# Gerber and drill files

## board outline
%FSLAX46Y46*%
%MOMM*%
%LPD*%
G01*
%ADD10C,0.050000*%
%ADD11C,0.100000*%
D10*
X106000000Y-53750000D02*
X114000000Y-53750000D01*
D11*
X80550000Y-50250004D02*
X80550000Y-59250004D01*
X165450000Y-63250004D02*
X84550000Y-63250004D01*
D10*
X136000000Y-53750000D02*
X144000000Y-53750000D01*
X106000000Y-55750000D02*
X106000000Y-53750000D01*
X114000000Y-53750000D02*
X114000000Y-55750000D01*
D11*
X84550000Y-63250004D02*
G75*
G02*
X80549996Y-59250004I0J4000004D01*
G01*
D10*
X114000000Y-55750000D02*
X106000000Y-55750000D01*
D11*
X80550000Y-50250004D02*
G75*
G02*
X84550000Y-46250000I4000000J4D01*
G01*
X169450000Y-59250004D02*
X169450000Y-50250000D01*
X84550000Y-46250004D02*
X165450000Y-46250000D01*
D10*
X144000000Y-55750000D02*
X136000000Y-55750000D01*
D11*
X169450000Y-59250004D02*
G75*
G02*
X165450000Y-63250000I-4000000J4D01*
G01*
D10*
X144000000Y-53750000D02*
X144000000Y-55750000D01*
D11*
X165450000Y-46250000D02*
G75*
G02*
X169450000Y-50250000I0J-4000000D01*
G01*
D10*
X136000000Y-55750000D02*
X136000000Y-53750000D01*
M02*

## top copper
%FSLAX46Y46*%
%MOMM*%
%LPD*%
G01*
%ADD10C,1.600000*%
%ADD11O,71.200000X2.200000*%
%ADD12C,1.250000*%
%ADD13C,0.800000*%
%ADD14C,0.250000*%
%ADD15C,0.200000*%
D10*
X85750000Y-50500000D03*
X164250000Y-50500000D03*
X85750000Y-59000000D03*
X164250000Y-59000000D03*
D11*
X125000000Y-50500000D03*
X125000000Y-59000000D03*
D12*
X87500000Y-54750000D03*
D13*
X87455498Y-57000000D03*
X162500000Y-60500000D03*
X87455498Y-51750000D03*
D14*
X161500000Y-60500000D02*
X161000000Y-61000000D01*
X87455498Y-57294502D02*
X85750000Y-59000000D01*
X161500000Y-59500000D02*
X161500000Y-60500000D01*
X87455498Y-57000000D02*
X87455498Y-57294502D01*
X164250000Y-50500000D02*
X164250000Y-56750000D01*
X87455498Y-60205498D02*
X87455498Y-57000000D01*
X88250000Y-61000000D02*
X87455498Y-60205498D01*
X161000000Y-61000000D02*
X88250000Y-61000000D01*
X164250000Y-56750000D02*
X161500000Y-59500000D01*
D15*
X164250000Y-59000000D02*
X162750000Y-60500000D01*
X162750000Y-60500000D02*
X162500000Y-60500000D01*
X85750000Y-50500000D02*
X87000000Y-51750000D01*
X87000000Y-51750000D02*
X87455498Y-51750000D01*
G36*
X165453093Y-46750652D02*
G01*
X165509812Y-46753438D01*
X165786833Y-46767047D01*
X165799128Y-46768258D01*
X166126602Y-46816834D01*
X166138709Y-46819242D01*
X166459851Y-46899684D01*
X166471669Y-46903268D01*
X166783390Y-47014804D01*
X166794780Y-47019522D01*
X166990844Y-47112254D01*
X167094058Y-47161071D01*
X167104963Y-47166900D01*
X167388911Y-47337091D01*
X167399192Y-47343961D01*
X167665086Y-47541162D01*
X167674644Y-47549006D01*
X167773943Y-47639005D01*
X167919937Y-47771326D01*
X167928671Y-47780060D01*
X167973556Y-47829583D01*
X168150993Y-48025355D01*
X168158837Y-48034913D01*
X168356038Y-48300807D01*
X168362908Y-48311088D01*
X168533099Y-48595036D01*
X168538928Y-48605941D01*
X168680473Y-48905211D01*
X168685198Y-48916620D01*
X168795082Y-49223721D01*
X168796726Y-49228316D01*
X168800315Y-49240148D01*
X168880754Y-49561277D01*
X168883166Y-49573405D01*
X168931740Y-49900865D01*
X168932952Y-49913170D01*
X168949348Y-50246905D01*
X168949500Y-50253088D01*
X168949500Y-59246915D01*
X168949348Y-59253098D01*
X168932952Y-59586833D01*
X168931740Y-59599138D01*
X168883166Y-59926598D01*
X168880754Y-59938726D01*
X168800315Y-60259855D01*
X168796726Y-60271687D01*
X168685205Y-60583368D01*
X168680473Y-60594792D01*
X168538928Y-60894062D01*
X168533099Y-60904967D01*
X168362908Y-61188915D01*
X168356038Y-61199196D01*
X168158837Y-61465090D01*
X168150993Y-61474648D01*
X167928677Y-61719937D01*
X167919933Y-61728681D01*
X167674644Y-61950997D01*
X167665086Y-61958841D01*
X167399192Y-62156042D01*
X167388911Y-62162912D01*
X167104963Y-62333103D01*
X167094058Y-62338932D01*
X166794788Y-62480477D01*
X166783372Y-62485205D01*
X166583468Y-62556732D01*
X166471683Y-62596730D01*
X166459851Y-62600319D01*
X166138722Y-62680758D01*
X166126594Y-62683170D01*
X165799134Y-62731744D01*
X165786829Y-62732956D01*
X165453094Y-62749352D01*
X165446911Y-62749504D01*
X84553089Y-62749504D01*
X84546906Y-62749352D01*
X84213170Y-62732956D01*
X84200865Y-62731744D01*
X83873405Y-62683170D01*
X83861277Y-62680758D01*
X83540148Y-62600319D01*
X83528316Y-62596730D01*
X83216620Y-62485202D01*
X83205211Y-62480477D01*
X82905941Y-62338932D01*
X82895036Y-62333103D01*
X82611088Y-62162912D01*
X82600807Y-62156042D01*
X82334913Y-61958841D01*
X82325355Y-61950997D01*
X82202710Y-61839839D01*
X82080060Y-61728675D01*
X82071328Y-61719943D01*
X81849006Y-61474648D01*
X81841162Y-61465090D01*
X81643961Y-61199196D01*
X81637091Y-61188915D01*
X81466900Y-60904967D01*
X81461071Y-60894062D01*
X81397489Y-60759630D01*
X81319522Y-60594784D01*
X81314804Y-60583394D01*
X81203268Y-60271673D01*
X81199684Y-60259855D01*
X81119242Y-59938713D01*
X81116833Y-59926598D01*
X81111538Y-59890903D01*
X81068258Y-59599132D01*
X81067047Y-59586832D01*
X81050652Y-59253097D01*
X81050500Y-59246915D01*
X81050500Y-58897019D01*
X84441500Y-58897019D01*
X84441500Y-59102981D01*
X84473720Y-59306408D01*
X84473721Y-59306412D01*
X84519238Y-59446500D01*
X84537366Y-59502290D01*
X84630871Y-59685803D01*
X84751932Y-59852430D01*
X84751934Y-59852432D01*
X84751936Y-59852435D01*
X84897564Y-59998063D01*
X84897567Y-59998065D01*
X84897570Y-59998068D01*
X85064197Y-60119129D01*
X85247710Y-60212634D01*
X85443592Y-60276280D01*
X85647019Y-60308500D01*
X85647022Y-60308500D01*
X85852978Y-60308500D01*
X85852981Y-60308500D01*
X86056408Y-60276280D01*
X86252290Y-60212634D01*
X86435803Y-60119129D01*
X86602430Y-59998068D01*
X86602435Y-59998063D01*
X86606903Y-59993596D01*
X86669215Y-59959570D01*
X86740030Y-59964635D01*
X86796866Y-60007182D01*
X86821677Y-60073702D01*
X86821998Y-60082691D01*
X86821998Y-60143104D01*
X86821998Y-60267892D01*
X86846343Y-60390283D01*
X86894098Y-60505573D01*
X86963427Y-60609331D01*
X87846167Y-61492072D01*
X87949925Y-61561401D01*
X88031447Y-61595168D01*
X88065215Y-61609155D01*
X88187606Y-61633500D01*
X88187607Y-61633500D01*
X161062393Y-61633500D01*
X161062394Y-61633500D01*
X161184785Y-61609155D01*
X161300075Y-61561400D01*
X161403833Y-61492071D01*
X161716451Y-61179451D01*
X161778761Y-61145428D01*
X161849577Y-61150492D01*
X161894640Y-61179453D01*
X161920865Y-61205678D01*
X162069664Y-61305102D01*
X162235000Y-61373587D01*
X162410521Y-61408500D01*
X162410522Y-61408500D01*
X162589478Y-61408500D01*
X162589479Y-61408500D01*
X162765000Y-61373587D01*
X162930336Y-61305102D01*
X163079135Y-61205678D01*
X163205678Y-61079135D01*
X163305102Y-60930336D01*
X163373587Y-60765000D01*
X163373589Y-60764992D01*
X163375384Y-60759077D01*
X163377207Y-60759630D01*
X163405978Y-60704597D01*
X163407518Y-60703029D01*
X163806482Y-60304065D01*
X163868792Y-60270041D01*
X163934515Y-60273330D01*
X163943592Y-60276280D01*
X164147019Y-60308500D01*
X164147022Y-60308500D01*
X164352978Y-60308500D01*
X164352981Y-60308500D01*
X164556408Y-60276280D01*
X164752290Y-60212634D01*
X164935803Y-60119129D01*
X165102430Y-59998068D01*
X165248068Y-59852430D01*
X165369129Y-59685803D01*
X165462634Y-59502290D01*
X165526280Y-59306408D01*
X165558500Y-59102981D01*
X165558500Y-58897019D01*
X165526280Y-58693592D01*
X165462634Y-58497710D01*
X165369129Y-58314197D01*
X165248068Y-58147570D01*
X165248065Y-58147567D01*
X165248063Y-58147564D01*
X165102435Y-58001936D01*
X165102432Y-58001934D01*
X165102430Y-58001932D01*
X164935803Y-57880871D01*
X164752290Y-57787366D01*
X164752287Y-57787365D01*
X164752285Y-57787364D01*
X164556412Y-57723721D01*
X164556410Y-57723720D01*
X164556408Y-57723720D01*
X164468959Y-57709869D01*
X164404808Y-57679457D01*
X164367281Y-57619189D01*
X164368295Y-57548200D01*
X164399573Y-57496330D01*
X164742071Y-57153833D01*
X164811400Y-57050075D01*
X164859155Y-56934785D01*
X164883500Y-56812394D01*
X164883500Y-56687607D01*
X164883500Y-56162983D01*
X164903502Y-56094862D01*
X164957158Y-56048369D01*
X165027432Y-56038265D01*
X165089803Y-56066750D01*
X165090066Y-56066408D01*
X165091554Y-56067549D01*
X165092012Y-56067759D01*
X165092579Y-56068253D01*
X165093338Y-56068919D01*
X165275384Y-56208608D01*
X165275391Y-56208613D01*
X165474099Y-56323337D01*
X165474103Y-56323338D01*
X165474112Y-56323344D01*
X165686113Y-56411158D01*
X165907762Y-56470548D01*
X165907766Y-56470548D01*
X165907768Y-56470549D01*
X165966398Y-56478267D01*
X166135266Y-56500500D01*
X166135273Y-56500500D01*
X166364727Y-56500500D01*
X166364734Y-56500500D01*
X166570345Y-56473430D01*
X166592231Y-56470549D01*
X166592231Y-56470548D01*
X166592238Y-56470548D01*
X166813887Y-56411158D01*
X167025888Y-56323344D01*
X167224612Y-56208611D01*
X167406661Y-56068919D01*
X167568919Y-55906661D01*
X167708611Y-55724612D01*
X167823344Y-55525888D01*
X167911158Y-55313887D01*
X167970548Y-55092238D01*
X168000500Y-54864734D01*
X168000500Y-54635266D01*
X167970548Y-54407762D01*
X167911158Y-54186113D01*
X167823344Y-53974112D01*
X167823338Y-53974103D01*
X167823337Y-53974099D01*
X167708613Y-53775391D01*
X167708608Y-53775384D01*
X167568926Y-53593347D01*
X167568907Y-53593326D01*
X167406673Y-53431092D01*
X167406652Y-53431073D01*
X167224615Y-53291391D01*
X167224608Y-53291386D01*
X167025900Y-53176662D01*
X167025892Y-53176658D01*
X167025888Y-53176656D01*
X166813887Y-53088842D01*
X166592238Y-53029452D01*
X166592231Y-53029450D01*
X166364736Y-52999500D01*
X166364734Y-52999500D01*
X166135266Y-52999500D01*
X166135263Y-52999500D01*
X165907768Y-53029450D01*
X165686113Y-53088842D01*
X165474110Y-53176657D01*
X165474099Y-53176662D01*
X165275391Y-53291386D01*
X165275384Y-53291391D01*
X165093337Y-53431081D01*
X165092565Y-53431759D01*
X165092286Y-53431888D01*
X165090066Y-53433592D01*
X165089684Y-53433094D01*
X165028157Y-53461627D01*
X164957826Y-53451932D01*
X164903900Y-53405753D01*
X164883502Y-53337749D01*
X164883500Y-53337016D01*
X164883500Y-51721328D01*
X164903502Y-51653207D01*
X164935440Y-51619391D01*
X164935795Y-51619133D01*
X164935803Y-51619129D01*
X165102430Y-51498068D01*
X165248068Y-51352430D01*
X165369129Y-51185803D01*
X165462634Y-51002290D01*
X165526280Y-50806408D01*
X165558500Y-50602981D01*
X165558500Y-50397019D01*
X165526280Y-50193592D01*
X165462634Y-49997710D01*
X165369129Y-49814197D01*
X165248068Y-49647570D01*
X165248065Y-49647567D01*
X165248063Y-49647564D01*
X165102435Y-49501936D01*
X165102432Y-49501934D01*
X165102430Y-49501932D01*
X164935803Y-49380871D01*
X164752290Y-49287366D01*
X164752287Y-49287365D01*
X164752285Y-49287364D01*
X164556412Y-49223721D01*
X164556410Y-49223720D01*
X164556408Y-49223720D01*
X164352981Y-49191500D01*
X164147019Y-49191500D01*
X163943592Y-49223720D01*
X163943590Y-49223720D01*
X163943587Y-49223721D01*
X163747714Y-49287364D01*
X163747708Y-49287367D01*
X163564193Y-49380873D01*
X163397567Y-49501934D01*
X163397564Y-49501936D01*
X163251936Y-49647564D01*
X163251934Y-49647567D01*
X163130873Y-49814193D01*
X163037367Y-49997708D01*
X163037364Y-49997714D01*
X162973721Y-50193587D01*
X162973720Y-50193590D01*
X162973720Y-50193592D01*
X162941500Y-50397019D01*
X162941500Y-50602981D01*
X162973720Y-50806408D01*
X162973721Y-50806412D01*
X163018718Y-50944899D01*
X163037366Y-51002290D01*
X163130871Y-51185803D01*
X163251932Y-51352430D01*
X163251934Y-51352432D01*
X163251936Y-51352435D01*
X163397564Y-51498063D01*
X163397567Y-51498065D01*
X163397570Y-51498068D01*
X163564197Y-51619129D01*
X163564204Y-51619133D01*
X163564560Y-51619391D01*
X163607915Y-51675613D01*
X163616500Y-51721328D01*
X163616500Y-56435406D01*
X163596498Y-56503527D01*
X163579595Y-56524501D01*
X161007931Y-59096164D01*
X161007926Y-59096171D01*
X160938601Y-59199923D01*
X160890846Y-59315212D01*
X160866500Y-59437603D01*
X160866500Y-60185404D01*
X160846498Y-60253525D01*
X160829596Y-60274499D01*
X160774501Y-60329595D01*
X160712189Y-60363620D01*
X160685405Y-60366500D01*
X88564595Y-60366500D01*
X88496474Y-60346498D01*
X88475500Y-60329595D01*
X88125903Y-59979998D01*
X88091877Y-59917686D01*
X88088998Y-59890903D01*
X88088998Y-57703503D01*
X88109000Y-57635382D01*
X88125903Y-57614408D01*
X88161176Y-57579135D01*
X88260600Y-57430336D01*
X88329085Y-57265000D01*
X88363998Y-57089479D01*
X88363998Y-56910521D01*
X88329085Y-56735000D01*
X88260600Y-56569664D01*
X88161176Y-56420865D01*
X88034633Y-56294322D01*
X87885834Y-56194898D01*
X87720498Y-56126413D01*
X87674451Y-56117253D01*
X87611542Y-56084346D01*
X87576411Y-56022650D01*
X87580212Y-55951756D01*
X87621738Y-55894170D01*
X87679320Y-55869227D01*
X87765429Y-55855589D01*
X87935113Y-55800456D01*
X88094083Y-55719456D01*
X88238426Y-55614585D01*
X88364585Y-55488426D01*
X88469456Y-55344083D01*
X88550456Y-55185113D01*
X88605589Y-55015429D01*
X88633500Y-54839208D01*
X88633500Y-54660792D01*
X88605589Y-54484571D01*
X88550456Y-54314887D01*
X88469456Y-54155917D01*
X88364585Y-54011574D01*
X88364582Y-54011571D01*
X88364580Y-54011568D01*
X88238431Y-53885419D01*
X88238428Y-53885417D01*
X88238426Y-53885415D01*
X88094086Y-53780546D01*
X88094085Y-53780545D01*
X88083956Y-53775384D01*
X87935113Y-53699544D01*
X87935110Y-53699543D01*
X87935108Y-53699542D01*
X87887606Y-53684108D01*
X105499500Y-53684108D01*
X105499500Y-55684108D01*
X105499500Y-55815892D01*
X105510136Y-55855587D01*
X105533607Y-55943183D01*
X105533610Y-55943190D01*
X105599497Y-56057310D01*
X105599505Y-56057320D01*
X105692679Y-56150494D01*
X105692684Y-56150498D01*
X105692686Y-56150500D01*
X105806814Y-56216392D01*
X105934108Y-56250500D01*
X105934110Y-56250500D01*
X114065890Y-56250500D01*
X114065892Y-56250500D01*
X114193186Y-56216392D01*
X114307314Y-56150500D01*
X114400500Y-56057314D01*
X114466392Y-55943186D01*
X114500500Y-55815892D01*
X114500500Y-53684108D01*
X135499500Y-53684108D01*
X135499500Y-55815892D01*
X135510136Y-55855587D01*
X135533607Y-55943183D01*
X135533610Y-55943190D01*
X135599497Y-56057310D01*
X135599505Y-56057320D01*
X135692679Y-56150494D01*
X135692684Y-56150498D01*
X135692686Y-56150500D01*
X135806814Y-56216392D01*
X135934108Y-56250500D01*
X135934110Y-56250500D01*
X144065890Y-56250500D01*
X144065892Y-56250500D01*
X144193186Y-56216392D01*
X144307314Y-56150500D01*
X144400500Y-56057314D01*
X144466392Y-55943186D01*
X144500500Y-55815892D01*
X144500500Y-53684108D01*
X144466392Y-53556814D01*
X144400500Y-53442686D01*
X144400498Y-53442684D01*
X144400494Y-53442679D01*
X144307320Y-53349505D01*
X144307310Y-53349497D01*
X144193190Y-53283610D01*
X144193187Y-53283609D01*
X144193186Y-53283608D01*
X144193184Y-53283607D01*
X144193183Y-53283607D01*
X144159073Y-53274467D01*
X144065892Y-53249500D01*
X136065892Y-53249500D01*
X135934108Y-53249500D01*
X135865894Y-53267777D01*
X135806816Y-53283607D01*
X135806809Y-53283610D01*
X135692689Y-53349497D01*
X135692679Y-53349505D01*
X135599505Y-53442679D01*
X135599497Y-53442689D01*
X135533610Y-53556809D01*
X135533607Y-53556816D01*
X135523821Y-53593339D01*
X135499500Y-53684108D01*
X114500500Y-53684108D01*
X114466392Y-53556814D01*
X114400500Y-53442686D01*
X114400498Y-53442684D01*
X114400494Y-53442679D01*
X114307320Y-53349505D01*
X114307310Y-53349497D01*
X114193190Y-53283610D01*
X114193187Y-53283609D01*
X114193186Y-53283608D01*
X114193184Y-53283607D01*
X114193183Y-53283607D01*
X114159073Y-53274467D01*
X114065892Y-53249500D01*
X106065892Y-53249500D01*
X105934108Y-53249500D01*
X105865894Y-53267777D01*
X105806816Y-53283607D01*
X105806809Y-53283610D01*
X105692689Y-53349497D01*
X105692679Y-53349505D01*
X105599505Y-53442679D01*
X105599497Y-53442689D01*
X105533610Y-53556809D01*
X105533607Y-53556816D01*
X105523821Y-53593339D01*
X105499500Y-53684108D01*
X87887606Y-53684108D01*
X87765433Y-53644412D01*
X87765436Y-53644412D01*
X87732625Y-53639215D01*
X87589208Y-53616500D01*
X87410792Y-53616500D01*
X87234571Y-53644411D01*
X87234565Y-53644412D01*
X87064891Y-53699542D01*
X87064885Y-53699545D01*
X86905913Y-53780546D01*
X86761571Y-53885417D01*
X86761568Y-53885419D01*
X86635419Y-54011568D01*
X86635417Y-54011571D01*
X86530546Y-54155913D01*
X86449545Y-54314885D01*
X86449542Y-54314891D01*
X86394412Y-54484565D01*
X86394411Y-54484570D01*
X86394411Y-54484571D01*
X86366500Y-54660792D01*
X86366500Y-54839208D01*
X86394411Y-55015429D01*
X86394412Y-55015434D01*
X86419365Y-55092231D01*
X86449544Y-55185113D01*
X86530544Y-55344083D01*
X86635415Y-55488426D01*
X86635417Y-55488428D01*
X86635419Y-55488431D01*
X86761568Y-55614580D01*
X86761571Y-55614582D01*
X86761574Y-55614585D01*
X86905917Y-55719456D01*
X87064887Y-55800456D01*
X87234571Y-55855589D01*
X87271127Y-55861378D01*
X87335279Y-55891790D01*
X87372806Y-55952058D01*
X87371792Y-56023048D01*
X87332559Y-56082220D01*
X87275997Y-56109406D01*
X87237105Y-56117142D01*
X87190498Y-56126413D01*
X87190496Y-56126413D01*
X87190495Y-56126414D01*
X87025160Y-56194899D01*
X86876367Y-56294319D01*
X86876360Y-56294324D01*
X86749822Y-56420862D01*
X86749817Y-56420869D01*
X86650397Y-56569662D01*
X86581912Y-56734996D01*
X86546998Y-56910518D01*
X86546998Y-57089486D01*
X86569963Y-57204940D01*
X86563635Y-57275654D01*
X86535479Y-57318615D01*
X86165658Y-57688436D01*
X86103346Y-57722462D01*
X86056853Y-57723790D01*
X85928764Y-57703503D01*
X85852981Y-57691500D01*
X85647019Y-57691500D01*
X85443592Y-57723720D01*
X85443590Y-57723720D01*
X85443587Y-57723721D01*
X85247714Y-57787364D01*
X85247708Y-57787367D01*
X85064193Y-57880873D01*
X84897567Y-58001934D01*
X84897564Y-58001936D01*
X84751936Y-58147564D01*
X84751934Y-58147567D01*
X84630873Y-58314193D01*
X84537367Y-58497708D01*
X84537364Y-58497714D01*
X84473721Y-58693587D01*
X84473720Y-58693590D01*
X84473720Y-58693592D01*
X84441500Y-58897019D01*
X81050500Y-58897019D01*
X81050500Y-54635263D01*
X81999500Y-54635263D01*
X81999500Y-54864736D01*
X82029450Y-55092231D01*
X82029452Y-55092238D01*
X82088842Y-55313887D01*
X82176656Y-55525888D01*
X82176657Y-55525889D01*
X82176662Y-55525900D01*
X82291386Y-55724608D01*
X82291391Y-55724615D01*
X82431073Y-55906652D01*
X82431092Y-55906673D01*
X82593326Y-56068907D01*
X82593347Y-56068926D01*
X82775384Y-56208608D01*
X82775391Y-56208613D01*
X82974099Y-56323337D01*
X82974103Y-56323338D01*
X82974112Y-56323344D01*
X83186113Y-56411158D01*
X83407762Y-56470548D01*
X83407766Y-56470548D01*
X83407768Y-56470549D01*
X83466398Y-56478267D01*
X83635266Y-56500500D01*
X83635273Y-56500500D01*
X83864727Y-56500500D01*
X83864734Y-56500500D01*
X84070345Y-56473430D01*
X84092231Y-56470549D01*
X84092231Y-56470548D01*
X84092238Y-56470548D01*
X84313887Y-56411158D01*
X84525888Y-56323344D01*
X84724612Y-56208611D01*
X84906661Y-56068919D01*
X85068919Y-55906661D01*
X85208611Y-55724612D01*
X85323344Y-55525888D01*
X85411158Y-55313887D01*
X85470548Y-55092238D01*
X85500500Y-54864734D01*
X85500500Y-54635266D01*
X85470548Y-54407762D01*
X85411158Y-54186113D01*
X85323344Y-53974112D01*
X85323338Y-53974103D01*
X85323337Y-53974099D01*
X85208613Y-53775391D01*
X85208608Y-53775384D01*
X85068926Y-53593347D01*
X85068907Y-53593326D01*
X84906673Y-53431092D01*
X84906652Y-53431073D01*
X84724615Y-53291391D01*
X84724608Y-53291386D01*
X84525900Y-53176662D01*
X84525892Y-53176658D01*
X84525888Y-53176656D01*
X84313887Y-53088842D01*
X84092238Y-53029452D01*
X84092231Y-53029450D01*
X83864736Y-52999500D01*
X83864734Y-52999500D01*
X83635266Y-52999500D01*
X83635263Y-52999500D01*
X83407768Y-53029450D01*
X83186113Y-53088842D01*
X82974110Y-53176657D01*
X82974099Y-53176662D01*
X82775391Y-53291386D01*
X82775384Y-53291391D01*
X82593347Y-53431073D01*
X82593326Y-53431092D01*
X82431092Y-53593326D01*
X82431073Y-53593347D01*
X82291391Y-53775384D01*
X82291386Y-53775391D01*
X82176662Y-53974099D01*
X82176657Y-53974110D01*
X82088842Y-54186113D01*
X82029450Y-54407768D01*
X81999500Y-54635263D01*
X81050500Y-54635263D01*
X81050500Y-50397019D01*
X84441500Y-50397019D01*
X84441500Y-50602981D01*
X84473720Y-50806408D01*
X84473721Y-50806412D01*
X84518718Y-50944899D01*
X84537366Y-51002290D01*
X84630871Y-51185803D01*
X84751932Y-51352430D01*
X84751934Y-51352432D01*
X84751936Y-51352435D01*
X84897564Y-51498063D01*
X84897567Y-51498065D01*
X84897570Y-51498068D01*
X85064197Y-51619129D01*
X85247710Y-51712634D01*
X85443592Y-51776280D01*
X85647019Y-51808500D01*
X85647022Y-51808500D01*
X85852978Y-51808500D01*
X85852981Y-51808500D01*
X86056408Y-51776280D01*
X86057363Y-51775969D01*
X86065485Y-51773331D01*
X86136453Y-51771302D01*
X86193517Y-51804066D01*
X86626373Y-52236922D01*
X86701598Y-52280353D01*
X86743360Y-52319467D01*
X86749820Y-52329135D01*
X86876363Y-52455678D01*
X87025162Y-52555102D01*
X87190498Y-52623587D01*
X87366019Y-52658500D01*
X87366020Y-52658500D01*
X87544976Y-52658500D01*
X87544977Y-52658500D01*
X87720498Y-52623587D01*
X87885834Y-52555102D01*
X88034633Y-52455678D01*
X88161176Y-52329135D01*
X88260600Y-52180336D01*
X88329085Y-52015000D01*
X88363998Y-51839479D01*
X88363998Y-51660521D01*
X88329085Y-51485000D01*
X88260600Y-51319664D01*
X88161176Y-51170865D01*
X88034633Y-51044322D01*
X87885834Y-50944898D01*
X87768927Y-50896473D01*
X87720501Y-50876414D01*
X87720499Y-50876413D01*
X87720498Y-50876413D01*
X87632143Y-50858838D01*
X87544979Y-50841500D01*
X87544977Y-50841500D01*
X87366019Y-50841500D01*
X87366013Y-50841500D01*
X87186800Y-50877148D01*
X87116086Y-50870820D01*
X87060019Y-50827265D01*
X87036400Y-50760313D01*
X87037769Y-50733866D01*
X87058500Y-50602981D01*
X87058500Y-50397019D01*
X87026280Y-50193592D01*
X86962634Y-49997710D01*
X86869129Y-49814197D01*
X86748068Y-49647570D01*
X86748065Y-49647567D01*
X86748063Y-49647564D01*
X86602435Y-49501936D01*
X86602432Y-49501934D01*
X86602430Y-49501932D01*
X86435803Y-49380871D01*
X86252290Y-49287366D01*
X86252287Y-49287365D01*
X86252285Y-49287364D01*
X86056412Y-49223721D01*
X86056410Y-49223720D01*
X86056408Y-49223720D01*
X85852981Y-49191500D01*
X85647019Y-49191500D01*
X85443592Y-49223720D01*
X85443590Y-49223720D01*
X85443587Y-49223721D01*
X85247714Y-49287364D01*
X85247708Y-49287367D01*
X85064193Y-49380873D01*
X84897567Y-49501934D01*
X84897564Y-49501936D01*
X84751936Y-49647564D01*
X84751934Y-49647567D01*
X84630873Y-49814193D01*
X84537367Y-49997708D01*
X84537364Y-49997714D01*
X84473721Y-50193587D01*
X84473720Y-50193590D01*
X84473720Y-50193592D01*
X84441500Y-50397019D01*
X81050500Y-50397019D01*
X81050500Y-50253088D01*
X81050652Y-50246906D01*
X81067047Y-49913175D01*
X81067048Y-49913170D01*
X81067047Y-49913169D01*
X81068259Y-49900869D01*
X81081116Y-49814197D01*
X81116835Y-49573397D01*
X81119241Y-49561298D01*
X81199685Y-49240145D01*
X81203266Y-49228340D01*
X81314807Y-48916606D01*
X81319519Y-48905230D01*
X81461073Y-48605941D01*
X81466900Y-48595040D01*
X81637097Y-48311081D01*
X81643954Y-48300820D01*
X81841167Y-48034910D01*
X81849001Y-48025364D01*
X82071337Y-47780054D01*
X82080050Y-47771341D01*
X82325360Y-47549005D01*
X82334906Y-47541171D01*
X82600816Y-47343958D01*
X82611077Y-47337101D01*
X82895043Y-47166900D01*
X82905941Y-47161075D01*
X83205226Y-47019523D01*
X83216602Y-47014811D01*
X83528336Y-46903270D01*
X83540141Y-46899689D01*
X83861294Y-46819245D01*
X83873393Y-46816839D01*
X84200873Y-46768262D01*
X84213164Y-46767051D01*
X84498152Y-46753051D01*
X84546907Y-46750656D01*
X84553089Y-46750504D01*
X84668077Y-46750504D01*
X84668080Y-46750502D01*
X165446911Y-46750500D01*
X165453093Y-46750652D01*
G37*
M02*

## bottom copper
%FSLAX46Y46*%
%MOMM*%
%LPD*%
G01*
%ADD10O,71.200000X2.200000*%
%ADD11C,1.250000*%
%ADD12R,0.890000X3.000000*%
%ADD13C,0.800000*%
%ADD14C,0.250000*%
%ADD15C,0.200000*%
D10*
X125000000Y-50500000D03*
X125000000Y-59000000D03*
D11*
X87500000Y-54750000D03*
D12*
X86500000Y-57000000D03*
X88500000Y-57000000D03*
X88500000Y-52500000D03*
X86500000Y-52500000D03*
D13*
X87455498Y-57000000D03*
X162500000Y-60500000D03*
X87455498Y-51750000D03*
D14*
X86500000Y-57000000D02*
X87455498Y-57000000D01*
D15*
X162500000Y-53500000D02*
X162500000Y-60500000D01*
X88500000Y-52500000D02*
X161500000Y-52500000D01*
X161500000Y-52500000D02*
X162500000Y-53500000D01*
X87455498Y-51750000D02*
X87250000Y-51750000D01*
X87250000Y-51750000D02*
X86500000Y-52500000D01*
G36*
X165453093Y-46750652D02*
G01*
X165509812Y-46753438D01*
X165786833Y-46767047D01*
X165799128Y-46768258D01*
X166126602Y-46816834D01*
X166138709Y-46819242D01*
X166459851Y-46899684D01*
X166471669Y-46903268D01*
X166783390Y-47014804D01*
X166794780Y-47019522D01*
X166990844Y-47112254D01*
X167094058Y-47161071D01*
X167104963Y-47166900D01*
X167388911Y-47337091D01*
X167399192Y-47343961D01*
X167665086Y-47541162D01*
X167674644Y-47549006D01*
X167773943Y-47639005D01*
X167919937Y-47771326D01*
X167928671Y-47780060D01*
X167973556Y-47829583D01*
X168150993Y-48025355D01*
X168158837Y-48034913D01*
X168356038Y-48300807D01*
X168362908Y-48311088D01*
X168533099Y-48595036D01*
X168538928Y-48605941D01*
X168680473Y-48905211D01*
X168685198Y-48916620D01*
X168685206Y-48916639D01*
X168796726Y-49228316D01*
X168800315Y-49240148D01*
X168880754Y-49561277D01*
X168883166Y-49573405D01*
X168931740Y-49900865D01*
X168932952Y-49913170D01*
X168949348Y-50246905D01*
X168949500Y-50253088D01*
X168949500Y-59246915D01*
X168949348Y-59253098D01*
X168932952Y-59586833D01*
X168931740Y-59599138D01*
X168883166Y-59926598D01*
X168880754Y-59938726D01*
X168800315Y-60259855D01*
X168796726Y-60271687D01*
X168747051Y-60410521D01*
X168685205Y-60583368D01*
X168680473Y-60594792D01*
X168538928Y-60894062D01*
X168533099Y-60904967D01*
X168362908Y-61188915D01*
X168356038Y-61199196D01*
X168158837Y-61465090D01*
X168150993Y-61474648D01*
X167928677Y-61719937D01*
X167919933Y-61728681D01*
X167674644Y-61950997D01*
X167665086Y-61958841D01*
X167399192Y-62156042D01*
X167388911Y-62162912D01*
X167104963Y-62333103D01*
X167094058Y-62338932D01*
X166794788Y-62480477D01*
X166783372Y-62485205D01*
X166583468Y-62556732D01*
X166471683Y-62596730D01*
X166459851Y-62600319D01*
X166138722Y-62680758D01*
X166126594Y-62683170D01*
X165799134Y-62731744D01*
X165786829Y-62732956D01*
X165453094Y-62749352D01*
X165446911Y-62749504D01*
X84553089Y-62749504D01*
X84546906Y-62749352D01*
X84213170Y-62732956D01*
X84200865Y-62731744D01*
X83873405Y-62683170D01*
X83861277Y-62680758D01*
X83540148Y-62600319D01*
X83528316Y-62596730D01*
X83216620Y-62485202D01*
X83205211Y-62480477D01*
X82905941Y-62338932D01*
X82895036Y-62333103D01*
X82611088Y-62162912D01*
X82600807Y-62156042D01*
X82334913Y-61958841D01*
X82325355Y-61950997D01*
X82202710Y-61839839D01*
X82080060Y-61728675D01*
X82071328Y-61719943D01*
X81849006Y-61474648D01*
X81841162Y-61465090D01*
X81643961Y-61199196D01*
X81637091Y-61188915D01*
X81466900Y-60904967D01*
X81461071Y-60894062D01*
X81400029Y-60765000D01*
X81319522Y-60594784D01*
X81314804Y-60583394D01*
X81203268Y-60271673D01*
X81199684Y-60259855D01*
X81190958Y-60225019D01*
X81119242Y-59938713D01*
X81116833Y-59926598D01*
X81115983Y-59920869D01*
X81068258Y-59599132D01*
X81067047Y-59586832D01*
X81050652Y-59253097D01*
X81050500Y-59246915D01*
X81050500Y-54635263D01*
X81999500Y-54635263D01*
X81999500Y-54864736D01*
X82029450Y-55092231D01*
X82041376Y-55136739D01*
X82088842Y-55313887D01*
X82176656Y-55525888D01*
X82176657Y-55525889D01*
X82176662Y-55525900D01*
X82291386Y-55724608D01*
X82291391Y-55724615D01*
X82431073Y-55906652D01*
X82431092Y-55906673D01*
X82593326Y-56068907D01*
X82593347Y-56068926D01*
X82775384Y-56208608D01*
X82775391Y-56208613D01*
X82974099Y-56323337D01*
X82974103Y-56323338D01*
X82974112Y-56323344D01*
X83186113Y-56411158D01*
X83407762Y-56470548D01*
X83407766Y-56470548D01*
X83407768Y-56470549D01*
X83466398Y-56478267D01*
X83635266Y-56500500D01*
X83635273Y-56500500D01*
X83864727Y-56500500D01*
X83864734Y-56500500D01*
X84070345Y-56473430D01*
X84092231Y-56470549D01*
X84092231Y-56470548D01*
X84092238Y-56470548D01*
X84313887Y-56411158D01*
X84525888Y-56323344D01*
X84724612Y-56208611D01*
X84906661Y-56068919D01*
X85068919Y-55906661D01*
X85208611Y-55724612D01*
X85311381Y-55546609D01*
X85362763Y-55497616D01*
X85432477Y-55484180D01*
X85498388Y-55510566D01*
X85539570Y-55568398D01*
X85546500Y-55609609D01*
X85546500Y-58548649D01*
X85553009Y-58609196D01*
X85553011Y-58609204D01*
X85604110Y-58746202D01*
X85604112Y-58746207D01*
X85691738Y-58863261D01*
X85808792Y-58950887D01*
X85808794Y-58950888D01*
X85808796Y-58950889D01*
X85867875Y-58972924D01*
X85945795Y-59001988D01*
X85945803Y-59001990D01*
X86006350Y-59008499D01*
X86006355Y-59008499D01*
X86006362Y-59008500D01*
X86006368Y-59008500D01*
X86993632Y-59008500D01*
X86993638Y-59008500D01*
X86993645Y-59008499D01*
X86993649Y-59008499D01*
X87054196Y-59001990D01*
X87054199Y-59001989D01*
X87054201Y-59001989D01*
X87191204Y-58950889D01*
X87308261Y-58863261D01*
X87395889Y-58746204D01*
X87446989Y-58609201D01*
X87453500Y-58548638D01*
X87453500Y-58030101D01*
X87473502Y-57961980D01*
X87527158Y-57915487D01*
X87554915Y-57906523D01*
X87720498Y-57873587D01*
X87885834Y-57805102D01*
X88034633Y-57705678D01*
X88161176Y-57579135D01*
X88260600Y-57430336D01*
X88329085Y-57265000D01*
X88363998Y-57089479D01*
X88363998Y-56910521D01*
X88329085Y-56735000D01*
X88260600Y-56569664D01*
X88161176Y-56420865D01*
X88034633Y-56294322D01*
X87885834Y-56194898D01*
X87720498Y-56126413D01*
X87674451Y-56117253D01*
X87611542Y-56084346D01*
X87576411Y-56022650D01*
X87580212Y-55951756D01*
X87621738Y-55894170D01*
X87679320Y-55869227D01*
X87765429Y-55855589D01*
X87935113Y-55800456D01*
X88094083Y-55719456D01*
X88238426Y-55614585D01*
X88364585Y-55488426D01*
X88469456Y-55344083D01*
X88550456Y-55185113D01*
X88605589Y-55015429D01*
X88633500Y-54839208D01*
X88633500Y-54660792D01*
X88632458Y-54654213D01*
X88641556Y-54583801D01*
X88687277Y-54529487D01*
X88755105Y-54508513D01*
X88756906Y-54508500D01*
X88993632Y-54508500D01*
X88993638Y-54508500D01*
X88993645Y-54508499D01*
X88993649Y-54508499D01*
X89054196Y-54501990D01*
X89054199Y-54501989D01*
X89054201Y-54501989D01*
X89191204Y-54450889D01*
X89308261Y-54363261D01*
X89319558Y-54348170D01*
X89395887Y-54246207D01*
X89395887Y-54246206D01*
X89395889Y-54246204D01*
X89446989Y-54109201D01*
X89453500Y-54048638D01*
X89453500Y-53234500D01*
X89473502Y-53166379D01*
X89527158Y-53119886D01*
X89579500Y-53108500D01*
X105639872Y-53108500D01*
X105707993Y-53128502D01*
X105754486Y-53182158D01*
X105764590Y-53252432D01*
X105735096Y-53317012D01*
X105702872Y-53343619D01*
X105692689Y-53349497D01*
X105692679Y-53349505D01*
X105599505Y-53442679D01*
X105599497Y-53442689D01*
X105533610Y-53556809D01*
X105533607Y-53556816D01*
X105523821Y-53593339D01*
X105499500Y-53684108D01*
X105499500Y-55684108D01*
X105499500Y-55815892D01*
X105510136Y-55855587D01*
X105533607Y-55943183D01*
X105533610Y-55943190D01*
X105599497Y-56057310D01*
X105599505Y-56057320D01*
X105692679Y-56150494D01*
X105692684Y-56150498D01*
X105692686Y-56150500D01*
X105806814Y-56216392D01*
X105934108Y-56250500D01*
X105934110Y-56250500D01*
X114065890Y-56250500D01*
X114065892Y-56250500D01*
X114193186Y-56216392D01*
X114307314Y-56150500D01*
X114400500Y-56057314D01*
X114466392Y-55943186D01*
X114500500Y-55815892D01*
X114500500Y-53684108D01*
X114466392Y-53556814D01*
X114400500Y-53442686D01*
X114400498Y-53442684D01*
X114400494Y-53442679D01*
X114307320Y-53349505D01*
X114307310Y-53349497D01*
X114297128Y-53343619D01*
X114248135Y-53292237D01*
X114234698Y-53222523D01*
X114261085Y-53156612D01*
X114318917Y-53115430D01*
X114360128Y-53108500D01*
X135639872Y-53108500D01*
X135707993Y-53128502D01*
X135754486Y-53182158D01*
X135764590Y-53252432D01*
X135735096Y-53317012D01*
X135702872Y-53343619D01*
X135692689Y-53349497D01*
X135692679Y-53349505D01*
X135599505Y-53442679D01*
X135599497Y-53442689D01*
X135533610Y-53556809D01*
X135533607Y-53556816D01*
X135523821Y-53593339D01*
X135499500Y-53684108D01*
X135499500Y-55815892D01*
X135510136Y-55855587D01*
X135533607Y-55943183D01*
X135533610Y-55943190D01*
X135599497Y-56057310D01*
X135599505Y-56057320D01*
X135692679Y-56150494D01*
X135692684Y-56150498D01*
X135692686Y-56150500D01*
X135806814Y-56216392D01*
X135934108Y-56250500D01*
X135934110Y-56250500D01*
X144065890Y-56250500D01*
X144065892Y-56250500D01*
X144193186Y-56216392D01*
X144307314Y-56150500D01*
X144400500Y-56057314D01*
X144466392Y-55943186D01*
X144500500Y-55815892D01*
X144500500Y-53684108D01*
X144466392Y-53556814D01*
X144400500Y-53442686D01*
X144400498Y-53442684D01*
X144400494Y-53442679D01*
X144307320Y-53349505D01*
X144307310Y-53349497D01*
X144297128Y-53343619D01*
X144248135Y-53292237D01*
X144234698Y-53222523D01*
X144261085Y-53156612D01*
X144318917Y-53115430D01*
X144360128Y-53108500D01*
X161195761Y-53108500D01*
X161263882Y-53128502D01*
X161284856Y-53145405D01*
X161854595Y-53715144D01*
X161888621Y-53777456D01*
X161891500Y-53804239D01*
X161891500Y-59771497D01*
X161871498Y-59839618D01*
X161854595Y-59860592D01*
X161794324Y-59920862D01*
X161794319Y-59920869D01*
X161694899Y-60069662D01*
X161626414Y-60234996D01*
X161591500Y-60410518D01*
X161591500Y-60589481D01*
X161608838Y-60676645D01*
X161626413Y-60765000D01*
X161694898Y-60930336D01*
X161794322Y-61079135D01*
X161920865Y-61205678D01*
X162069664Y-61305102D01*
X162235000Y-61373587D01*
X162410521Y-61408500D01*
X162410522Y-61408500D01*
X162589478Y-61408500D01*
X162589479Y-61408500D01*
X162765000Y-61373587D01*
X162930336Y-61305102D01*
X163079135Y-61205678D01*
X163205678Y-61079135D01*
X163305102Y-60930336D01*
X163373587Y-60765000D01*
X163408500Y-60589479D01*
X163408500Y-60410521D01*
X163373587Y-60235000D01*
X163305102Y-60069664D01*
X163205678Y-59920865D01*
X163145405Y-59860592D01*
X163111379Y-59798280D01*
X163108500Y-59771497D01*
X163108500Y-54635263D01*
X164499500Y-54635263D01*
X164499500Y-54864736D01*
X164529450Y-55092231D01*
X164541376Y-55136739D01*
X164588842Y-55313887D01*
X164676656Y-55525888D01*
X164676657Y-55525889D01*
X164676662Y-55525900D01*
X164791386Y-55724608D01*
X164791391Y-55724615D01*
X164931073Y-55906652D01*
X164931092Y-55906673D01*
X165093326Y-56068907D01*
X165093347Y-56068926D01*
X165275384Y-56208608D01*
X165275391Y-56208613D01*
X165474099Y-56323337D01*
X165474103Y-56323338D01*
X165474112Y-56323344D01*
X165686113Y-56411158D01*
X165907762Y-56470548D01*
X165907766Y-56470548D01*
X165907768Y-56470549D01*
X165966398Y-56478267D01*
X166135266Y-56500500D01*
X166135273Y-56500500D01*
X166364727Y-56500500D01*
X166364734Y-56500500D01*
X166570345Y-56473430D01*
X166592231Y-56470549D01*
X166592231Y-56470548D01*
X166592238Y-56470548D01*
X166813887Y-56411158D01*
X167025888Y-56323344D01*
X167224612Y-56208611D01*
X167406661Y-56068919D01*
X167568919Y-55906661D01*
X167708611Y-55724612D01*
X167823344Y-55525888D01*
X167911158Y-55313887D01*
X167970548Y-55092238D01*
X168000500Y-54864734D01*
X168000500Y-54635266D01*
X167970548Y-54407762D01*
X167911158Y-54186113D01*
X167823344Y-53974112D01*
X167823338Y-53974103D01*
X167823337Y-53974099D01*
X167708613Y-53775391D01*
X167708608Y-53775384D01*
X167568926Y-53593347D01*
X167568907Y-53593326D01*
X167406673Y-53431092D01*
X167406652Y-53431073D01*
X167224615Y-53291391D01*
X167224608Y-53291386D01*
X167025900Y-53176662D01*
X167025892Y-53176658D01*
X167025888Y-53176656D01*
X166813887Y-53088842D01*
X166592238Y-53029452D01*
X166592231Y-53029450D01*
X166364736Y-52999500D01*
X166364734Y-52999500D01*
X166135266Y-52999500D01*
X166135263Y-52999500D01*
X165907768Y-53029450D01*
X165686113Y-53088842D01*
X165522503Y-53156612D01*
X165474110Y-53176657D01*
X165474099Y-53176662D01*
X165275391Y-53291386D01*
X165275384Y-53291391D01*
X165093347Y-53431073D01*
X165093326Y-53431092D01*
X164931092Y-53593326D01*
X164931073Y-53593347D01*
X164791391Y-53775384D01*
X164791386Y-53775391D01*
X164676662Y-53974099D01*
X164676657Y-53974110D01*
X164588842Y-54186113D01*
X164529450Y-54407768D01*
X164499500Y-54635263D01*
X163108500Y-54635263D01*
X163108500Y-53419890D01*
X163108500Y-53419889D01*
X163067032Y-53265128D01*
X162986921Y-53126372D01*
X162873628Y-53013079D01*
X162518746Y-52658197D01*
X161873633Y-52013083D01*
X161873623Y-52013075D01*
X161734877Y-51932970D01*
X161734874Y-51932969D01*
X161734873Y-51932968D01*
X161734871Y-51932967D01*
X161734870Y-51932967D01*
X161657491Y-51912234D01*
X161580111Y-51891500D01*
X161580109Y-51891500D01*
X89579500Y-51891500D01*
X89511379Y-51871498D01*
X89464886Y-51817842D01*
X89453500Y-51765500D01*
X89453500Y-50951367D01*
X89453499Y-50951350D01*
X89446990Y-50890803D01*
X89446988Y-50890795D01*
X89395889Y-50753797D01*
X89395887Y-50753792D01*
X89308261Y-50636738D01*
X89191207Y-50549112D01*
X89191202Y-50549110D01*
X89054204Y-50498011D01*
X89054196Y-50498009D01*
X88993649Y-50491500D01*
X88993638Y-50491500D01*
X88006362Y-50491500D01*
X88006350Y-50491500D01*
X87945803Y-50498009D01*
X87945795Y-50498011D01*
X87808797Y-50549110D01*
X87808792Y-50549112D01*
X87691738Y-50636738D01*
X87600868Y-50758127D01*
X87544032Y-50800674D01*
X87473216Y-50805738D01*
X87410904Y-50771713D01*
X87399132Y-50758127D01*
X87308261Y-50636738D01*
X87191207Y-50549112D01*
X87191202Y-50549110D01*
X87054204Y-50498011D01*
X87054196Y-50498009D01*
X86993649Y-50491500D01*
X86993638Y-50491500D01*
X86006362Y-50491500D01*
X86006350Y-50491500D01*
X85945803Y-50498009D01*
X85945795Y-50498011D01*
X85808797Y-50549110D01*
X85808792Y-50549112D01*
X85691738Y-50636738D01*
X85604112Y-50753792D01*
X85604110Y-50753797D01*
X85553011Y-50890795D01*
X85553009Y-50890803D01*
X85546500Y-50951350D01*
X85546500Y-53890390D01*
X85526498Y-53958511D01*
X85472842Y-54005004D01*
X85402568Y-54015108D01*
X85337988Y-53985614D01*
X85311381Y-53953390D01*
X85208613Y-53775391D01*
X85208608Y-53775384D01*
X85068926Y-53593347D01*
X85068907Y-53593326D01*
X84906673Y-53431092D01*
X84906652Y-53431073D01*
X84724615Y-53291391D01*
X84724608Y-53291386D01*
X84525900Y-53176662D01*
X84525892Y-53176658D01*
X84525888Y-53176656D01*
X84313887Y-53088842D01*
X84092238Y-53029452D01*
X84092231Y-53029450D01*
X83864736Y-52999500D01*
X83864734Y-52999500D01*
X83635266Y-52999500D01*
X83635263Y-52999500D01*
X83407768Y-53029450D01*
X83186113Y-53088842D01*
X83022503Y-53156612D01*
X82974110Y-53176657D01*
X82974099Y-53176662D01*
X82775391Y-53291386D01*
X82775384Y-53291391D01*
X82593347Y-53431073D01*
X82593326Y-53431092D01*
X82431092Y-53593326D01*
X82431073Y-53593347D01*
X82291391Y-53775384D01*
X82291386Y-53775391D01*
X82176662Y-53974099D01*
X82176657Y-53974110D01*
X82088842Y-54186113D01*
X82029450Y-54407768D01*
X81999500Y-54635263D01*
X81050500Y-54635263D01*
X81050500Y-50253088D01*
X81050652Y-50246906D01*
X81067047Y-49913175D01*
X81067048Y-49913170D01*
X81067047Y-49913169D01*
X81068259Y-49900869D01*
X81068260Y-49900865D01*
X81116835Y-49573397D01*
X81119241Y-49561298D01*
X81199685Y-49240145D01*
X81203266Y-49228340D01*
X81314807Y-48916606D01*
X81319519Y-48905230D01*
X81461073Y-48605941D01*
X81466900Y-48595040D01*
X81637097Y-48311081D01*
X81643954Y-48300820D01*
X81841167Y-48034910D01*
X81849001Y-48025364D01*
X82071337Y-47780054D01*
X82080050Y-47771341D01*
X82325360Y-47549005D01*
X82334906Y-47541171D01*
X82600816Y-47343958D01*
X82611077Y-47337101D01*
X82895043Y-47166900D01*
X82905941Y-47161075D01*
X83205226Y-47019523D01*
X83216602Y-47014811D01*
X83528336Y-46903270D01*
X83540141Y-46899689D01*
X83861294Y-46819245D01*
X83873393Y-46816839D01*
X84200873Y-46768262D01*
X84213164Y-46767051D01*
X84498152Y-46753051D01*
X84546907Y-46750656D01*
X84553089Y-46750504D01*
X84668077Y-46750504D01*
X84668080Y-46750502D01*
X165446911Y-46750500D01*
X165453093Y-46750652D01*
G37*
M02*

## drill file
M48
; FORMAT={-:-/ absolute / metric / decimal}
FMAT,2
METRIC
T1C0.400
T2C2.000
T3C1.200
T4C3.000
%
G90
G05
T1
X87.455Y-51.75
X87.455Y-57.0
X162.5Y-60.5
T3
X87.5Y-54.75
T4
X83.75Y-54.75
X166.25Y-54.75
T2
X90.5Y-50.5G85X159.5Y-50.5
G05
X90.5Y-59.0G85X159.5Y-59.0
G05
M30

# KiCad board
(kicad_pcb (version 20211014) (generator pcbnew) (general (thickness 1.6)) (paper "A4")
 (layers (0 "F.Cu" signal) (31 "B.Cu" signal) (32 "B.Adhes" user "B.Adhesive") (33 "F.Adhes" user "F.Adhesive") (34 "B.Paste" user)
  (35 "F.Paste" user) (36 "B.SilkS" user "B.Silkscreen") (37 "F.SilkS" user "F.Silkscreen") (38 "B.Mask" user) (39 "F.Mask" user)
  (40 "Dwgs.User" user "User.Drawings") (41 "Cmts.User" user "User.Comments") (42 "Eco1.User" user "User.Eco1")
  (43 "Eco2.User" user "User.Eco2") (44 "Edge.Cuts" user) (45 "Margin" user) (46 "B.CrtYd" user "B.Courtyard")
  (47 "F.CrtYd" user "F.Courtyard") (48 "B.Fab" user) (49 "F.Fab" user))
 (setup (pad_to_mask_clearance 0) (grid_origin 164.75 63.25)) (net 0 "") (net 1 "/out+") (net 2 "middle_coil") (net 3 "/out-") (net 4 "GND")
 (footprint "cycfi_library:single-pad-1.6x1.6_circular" (layer "F.Cu") (at 85.75 50.5)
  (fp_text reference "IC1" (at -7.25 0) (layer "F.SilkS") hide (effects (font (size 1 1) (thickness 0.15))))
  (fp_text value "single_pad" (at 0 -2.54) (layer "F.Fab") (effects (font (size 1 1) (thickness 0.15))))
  (pad "1" smd circle (at 0 0) (size 1.6 1.6) (layers "F.Cu" "F.Paste" "F.Mask") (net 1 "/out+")))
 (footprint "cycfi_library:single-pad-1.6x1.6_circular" (layer "F.Cu") (at 164.25 50.5)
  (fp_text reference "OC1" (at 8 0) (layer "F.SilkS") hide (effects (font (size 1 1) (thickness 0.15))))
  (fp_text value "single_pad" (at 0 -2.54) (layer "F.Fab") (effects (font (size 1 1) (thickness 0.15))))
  (pad "1" smd circle (at 0 0) (size 1.6 1.6) (layers "F.Cu" "F.Paste" "F.Mask") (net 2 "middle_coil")))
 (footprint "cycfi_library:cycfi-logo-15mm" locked (layer "F.Cu") (at 124.75 54.75)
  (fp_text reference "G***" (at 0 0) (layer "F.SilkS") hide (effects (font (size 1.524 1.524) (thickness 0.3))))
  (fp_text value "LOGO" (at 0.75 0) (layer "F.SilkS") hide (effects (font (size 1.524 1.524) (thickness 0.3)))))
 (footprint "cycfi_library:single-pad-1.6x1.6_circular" (layer "F.Cu") (at 85.75 59)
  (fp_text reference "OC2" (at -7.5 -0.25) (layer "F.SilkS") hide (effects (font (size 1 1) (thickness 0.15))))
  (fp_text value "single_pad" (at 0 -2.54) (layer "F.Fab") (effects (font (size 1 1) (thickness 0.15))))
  (pad "1" smd circle (at 0 0) (size 1.6 1.6) (layers "F.Cu" "F.Paste" "F.Mask") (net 2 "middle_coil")))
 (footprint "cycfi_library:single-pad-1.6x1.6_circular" (layer "F.Cu") (at 164.25 59)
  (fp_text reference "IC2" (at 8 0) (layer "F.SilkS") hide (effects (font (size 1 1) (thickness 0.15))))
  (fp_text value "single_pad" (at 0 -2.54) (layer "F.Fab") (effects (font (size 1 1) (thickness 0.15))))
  (pad "1" smd circle (at 0 0) (size 1.6 1.6) (layers "F.Cu" "F.Paste" "F.Mask") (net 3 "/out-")))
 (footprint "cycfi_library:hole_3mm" (layer "F.Cu") (at 166.25 54.75 180)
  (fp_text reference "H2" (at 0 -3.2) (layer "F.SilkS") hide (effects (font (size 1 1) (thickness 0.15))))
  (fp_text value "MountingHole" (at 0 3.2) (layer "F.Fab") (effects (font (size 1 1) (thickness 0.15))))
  (pad "" np_thru_hole circle (at 0 0 180) (size 3 3) (drill 3) (layers F&B.Cu *.Mask)))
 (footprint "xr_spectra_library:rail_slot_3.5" (layer "F.Cu") (at 125 50.5)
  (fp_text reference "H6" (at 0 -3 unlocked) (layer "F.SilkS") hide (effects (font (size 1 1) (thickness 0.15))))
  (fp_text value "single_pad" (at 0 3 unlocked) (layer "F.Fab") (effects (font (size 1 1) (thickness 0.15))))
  (pad "1" thru_hole oval (at 0 0) (size 71.2 2.2) (drill oval 71 2) (layers *.Cu *.Mask) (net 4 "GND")))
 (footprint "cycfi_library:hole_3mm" (layer "F.Cu") (at 83.75 54.75 180)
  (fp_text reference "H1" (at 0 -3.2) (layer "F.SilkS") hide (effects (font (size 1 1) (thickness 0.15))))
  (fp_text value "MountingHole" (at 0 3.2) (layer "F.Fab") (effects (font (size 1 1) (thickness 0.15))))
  (pad "" np_thru_hole circle (at 0 0 180) (size 3 3) (drill 3) (layers F&B.Cu *.Mask)))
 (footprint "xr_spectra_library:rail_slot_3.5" (layer "F.Cu") (at 125 59)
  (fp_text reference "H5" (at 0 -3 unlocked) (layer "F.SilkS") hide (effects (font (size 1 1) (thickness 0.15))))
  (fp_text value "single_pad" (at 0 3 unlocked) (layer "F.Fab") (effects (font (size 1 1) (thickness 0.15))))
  (pad "1" thru_hole oval (at 0 0) (size 71.2 2.2) (drill oval 71 2) (layers *.Cu *.Mask) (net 4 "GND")))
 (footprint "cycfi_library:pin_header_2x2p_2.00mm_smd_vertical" (layer "B.Cu") (at 87.5 54.75 -90)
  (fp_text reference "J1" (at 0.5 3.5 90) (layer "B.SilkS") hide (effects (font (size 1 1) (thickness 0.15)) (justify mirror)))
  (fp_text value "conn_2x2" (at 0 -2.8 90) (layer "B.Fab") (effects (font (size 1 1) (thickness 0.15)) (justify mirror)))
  (pad "" np_thru_hole circle (at 0 0 270) (size 1.25 1.25) (drill 1.2) (layers F&B.Cu *.Mask))
  (pad "1" smd rect (at 2.25 1 270) (size 3 0.89) (layers "B.Cu" "B.Paste" "B.Mask") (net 2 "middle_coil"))
  (pad "2" smd rect (at 2.25 -1 270) (size 3 0.89) (layers "B.Cu" "B.Paste" "B.Mask") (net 4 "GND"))
  (pad "3" smd rect (at -2.25 -1 270) (size 3 0.89) (layers "B.Cu" "B.Paste" "B.Mask") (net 3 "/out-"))
  (pad "4" smd rect (at -2.25 1 270) (size 3 0.89) (layers "B.Cu" "B.Paste" "B.Mask") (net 1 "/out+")))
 (gr_line (start 106 53.75) (end 114 53.75) (layer "Edge.Cuts") (width 0.05))
 (gr_line (start 80.55 50.250004) (end 80.55 59.250004) (layer "Edge.Cuts") (width 0.1))
 (gr_line (start 165.45 63.250004) (end 84.55 63.250004) (layer "Edge.Cuts") (width 0.1))
 (gr_line (start 136 53.75) (end 144 53.75) (layer "Edge.Cuts") (width 0.05))
 (gr_line (start 106 55.75) (end 106 53.75) (layer "Edge.Cuts") (width 0.05))
 (gr_line (start 114 53.75) (end 114 55.75) (layer "Edge.Cuts") (width 0.05))
 (gr_arc (start 84.55 63.250004) (mid 81.721573 62.078431) (end 80.55 59.250004) (layer "Edge.Cuts") (width 0.1))
 (gr_line (start 114 55.75) (end 106 55.75) (layer "Edge.Cuts") (width 0.05))
 (gr_arc (start 80.55 50.250004) (mid 81.721573 47.421577) (end 84.55 46.250004) (layer "Edge.Cuts") (width 0.1))
 (gr_line (start 169.45 59.250004) (end 169.45 50.25) (layer "Edge.Cuts") (width 0.1))
 (gr_line (start 84.55 46.250004) (end 165.45 46.25) (layer "Edge.Cuts") (width 0.1))
 (gr_line (start 144 55.75) (end 136 55.75) (layer "Edge.Cuts") (width 0.05))
 (gr_arc (start 169.45 59.250004) (mid 168.278427 62.078431) (end 165.45 63.250004) (layer "Edge.Cuts") (width 0.1))
 (gr_line (start 144 53.75) (end 144 55.75) (layer "Edge.Cuts") (width 0.05))
 (gr_arc (start 165.45 46.25) (mid 168.278427 47.421573) (end 169.45 50.25) (layer "Edge.Cuts") (width 0.1))
 (gr_line (start 136 55.75) (end 136 53.75) (layer "Edge.Cuts") (width 0.05))
 (segment (start 161.5 60.5) (end 161 61) (width 0.25) (layer "F.Cu") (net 2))
 (segment (start 87.455498 57.294502) (end 85.75 59) (width 0.25) (layer "F.Cu") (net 2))
 (segment (start 161.5 59.5) (end 161.5 60.5) (width 0.25) (layer "F.Cu") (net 2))
 (segment (start 87.455498 57) (end 87.455498 57.294502) (width 0.25) (layer "F.Cu") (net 2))
 (segment (start 164.25 50.5) (end 164.25 56.75) (width 0.25) (layer "F.Cu") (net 2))
 (segment (start 87.455498 60.205498) (end 87.455498 57) (width 0.25) (layer "F.Cu") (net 2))
 (segment (start 88.25 61) (end 87.455498 60.205498) (width 0.25) (layer "F.Cu") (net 2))
 (segment (start 161 61) (end 88.25 61) (width 0.25) (layer "F.Cu") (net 2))
 (segment (start 164.25 56.75) (end 161.5 59.5) (width 0.25) (layer "F.Cu") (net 2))
 (via (at 87.455498 57) (size 0.8) (drill 0.4) (layers "F.Cu" "B.Cu") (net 2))
 (segment (start 86.5 57) (end 87.455498 57) (width 0.25) (layer "B.Cu") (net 2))
 (segment (start 164.25 59) (end 162.75 60.5) (width 0.2) (layer "F.Cu") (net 3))
 (segment (start 162.75 60.5) (end 162.5 60.5) (width 0.2) (layer "F.Cu") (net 3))
 (via (at 162.5 60.5) (size 0.8) (drill 0.4) (layers "F.Cu" "B.Cu") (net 3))
 (segment (start 162.5 53.5) (end 162.5 60.5) (width 0.2) (layer "B.Cu") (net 3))
 (segment (start 88.5 52.5) (end 161.5 52.5) (width 0.2) (layer "B.Cu") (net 3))
 (segment (start 161.5 52.5) (end 162.5 53.5) (width 0.2) (layer "B.Cu") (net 3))
 (segment (start 85.75 50.5) (end 87 51.75) (width 0.2) (layer "F.Cu") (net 1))
 (segment (start 87 51.75) (end 87.455498 51.75) (width 0.2) (layer "F.Cu") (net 1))
 (via (at 87.455498 51.75) (size 0.8) (drill 0.4) (layers "F.Cu" "B.Cu") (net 1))
 (segment (start 87.455498 51.75) (end 87.25 51.75) (width 0.2) (layer "B.Cu") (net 1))
 (segment (start 87.25 51.75) (end 86.5 52.5) (width 0.2) (layer "B.Cu") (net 1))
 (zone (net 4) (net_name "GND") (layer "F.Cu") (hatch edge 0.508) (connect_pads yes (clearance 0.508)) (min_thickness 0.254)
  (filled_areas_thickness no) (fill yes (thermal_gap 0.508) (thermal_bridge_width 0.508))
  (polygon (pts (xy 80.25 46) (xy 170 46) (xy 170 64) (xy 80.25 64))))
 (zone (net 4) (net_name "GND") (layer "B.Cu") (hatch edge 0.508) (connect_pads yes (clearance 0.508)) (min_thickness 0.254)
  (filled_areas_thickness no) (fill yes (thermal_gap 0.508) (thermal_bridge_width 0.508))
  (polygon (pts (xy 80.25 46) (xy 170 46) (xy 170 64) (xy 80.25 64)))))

